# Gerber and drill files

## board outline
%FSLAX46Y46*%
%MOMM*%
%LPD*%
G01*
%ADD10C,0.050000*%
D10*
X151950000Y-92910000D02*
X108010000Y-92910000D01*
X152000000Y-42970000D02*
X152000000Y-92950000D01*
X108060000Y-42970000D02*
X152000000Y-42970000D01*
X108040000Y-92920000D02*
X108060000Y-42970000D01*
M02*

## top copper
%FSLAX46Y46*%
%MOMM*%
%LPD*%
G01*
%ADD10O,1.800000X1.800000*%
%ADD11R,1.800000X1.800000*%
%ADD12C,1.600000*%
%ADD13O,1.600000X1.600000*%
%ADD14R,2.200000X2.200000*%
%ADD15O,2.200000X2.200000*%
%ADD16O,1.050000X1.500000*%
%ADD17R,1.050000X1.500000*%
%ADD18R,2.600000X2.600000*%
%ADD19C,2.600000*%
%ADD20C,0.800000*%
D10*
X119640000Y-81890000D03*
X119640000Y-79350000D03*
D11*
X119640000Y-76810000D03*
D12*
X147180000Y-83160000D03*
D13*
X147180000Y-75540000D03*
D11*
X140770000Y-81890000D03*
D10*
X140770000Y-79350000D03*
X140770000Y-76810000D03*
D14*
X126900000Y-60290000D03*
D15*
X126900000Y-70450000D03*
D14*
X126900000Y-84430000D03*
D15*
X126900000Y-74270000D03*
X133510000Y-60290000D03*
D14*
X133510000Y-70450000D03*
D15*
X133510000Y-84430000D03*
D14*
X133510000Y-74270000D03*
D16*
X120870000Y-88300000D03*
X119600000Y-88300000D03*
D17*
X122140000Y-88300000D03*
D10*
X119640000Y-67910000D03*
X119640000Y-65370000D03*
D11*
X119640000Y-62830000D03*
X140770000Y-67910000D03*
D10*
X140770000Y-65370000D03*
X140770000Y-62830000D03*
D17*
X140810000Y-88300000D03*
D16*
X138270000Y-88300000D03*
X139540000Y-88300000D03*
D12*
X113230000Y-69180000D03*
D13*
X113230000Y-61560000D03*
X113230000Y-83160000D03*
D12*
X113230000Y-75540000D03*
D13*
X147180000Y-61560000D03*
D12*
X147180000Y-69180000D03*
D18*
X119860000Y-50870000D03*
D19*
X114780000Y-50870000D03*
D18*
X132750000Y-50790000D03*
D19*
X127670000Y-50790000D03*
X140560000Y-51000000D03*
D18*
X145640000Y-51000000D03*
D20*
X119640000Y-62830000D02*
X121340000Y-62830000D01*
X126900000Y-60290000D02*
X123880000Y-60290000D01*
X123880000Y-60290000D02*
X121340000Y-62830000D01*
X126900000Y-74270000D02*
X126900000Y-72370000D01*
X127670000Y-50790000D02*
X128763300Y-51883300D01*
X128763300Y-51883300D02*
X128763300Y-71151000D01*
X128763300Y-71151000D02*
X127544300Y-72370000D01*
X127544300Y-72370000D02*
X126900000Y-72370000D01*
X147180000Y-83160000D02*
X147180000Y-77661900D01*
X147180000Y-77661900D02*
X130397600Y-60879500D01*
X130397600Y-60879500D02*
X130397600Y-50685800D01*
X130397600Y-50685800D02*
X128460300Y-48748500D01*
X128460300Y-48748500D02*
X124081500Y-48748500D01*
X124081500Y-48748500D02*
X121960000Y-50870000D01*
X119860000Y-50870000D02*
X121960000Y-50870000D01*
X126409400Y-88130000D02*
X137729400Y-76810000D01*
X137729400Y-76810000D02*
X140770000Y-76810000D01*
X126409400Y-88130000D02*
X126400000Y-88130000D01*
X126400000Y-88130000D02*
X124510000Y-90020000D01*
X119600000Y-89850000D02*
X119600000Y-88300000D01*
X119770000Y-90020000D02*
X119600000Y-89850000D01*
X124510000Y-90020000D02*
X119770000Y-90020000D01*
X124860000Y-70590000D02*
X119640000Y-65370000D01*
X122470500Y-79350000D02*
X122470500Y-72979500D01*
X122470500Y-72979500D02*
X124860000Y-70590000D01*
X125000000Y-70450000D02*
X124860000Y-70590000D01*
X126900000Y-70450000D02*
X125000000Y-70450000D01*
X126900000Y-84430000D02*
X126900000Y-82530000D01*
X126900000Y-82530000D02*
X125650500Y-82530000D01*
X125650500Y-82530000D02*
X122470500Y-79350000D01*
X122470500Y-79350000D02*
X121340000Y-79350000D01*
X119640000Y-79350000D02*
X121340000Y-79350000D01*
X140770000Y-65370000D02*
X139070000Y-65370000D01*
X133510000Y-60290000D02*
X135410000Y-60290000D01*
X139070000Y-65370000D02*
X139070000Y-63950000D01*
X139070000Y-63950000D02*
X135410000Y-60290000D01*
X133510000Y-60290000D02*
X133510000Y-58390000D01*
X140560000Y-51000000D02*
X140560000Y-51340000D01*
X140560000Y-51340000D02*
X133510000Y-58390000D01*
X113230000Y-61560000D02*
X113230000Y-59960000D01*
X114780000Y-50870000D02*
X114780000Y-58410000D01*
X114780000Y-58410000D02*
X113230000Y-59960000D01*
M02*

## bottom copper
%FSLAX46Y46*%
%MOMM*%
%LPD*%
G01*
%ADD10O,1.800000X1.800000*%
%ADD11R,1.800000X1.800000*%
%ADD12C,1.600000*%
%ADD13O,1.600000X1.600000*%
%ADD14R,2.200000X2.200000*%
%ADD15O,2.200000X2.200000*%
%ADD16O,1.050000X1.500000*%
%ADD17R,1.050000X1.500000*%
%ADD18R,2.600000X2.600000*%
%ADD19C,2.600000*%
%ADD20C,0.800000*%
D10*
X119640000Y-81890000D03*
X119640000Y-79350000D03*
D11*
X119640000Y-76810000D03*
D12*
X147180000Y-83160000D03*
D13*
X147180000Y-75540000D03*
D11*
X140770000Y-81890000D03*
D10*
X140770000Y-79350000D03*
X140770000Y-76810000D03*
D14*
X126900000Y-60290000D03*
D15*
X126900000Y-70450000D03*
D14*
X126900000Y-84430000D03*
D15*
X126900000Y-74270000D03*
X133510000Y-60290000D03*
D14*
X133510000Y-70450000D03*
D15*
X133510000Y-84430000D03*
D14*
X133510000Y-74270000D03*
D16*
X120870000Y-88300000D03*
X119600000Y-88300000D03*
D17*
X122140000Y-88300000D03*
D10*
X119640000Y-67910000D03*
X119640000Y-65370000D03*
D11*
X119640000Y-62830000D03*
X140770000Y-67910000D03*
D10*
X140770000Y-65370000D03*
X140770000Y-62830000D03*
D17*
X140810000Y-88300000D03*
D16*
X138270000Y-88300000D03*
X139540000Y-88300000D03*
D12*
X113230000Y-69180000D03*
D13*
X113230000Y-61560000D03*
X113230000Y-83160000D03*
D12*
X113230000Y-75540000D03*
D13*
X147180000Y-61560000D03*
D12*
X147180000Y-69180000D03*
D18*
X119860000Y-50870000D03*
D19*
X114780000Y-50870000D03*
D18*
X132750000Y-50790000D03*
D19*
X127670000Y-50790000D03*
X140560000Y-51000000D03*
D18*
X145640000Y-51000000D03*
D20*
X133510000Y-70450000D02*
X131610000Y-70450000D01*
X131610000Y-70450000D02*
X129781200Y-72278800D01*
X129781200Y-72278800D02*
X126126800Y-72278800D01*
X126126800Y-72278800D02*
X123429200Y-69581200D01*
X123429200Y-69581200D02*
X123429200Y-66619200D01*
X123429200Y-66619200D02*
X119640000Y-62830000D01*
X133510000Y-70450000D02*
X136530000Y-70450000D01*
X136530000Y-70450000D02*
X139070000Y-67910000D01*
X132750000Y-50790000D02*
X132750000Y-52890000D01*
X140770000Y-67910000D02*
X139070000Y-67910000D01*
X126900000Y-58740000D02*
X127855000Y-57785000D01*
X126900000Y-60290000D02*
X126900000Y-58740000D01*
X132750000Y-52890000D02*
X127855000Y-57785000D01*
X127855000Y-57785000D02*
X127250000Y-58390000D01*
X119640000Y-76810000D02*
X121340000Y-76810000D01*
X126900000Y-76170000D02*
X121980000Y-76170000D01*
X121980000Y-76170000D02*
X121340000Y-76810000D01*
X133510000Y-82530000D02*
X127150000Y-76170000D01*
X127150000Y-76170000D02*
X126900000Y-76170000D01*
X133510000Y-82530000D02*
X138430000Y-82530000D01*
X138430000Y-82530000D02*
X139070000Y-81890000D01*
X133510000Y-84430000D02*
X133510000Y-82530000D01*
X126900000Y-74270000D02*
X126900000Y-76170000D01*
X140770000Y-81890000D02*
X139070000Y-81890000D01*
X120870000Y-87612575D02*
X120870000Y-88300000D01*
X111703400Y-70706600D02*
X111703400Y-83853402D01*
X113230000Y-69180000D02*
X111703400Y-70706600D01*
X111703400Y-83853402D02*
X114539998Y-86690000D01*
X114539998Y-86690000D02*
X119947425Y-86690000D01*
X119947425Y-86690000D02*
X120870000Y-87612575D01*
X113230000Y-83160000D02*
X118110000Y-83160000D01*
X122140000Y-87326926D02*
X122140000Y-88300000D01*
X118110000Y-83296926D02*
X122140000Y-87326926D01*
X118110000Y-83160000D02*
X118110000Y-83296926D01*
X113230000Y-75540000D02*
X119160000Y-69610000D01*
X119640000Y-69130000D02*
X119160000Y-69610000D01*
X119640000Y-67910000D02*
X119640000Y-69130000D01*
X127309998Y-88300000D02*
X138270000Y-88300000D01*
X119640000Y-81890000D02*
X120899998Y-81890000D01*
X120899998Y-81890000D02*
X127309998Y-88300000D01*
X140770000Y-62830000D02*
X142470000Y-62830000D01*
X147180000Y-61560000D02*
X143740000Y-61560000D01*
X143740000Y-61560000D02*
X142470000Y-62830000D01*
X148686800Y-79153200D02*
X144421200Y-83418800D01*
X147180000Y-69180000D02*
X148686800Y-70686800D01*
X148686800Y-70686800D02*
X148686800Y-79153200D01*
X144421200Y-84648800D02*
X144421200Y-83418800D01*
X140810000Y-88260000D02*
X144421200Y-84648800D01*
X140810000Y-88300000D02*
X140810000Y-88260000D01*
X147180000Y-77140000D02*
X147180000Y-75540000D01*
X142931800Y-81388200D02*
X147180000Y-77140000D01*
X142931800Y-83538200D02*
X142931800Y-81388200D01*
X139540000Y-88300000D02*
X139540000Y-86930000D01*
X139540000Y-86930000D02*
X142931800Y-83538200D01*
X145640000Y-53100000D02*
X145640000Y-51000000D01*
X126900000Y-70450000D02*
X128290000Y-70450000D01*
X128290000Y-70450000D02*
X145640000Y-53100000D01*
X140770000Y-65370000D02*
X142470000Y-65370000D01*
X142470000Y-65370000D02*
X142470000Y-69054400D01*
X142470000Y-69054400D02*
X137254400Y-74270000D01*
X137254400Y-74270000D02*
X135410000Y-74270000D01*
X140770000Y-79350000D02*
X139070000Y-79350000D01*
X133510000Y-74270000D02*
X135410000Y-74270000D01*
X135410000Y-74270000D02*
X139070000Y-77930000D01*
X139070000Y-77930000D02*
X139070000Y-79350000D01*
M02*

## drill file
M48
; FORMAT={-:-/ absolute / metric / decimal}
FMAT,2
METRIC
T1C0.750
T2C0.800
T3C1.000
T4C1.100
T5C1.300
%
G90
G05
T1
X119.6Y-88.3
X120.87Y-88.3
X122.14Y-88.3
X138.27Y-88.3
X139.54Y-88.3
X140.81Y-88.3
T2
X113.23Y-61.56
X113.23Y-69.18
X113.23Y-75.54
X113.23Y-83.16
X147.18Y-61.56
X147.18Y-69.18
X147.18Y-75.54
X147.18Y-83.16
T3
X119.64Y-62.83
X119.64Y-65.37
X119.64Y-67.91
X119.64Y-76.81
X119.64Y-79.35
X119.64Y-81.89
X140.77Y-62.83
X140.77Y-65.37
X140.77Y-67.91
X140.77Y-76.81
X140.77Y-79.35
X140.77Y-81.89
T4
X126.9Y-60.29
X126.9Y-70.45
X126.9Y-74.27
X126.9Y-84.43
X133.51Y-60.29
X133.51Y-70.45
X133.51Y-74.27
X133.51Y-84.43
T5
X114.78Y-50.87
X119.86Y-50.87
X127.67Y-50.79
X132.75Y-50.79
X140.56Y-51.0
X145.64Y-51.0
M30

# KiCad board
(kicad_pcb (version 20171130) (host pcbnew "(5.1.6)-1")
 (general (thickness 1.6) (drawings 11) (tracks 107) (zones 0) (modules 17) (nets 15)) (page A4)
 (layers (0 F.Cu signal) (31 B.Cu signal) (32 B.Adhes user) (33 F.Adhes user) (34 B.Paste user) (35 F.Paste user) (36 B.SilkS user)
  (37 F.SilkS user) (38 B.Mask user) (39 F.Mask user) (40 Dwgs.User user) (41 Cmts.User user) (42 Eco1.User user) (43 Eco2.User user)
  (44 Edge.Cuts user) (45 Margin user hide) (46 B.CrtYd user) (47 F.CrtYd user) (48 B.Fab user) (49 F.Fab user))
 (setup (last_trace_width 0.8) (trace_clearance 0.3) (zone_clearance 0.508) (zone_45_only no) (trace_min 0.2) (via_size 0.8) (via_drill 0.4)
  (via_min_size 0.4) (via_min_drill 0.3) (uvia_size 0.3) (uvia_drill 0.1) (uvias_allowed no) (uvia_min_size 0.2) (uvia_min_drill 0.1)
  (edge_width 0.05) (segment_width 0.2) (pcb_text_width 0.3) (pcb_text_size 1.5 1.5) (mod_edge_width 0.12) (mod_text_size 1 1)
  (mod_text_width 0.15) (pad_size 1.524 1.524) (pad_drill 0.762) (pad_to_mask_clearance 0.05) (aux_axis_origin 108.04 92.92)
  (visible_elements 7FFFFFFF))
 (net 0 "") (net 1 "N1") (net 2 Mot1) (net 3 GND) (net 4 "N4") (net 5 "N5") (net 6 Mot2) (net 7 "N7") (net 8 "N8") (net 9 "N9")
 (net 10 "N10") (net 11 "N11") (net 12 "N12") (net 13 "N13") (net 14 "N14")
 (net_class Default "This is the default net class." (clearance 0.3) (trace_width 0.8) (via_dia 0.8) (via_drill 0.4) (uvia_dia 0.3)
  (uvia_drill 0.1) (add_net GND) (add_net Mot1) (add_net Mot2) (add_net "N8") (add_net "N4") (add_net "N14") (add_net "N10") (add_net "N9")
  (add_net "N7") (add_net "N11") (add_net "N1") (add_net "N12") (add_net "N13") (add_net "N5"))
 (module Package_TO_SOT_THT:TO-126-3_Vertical (layer F.Cu) (at 119.64 76.81 270)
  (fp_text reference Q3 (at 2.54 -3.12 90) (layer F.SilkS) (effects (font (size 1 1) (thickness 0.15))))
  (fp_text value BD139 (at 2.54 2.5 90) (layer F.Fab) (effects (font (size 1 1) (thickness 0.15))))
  (pad 3 thru_hole oval (at 5.08 0 270) (size 1.8 1.8) (drill 1) (layers *.Cu *.Mask) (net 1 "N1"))
  (pad 2 thru_hole oval (at 2.54 0 270) (size 1.8 1.8) (drill 1) (layers *.Cu *.Mask) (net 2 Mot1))
  (pad 1 thru_hole rect (at 0 0 270) (size 1.8 1.8) (drill 1) (layers *.Cu *.Mask) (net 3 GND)))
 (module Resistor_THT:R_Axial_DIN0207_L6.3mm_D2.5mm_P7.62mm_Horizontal (layer F.Cu) (at 147.18 83.16 90)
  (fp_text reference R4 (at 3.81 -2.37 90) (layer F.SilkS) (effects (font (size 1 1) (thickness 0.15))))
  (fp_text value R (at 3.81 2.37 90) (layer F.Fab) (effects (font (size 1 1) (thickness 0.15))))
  (pad 1 thru_hole circle (at 0 0 90) (size 1.6 1.6) (drill 0.8) (layers *.Cu *.Mask) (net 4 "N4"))
  (pad 2 thru_hole oval (at 7.62 0 90) (size 1.6 1.6) (drill 0.8) (layers *.Cu *.Mask) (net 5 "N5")))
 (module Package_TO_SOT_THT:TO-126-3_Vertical (layer F.Cu) (at 140.77 81.89 90)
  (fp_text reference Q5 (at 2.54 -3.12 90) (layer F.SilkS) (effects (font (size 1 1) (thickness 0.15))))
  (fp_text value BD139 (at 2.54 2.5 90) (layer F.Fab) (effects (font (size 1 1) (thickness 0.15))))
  (pad 1 thru_hole rect (at 0 0 90) (size 1.8 1.8) (drill 1) (layers *.Cu *.Mask) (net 3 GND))
  (pad 2 thru_hole oval (at 2.54 0 90) (size 1.8 1.8) (drill 1) (layers *.Cu *.Mask) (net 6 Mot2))
  (pad 3 thru_hole oval (at 5.08 0 90) (size 1.8 1.8) (drill 1) (layers *.Cu *.Mask) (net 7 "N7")))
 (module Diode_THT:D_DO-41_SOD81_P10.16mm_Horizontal (layer F.Cu) (at 126.9 60.29 270)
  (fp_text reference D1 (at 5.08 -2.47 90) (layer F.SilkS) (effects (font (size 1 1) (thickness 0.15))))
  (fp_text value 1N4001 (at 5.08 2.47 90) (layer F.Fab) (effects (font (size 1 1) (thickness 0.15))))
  (pad 1 thru_hole rect (at 0 0 270) (size 2.2 2.2) (drill 1.1) (layers *.Cu *.Mask) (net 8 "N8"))
  (pad 2 thru_hole oval (at 10.16 0 270) (size 2.2 2.2) (drill 1.1) (layers *.Cu *.Mask) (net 2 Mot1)))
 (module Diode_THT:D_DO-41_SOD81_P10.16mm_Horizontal (layer F.Cu) (at 126.9 84.43 90)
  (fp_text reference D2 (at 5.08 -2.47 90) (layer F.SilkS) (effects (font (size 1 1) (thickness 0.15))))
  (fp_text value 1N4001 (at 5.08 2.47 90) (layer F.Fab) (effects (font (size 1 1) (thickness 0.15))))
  (pad 1 thru_hole rect (at 0 0 90) (size 2.2 2.2) (drill 1.1) (layers *.Cu *.Mask) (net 2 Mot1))
  (pad 2 thru_hole oval (at 10.16 0 90) (size 2.2 2.2) (drill 1.1) (layers *.Cu *.Mask) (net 3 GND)))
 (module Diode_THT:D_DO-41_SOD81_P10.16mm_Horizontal (layer F.Cu) (at 133.51 70.45 90)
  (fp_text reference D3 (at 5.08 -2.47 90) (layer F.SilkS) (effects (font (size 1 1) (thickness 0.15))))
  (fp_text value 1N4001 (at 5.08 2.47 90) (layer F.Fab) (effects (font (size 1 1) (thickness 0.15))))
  (pad 2 thru_hole oval (at 10.16 0 90) (size 2.2 2.2) (drill 1.1) (layers *.Cu *.Mask) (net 6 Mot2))
  (pad 1 thru_hole rect (at 0 0 90) (size 2.2 2.2) (drill 1.1) (layers *.Cu *.Mask) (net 8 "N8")))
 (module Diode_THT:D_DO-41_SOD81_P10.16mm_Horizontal (layer F.Cu) (at 133.51 74.27 270)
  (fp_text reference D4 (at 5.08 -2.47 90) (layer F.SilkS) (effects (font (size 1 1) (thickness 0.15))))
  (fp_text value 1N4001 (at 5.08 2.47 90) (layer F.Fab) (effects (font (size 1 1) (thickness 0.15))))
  (pad 2 thru_hole oval (at 10.16 0 270) (size 2.2 2.2) (drill 1.1) (layers *.Cu *.Mask) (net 3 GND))
  (pad 1 thru_hole rect (at 0 0 270) (size 2.2 2.2) (drill 1.1) (layers *.Cu *.Mask) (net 6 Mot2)))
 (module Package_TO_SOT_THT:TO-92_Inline (layer F.Cu) (at 122.14 88.3 180)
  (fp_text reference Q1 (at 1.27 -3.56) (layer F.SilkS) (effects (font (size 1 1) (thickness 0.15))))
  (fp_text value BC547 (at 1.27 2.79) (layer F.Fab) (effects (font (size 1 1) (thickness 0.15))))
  (pad 2 thru_hole oval (at 1.27 0 180) (size 1.05 1.5) (drill 0.75) (layers *.Cu *.Mask) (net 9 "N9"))
  (pad 3 thru_hole oval (at 2.54 0 180) (size 1.05 1.5) (drill 0.75) (layers *.Cu *.Mask) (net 7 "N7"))
  (pad 1 thru_hole rect (at 0 0 180) (size 1.05 1.5) (drill 0.75) (layers *.Cu *.Mask) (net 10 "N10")))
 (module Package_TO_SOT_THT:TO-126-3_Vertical (layer F.Cu) (at 119.64 62.83 270)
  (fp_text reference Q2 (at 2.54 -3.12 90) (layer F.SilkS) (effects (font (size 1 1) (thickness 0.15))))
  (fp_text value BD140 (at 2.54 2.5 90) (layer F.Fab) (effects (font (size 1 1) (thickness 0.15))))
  (pad 3 thru_hole oval (at 5.08 0 270) (size 1.8 1.8) (drill 1) (layers *.Cu *.Mask) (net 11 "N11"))
  (pad 2 thru_hole oval (at 2.54 0 270) (size 1.8 1.8) (drill 1) (layers *.Cu *.Mask) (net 2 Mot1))
  (pad 1 thru_hole rect (at 0 0 270) (size 1.8 1.8) (drill 1) (layers *.Cu *.Mask) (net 8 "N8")))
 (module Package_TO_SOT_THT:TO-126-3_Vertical (layer F.Cu) (at 140.77 67.91 90)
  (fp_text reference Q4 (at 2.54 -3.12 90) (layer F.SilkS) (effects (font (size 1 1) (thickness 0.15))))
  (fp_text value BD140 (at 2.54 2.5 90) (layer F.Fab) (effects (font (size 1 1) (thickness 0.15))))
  (pad 1 thru_hole rect (at 0 0 90) (size 1.8 1.8) (drill 1) (layers *.Cu *.Mask) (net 8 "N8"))
  (pad 2 thru_hole oval (at 2.54 0 90) (size 1.8 1.8) (drill 1) (layers *.Cu *.Mask) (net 6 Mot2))
  (pad 3 thru_hole oval (at 5.08 0 90) (size 1.8 1.8) (drill 1) (layers *.Cu *.Mask) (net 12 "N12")))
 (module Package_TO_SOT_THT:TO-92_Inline (layer F.Cu) (at 140.81 88.3 180)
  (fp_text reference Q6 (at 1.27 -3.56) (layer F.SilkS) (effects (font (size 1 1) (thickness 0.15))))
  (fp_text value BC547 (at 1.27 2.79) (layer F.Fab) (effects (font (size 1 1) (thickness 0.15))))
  (pad 1 thru_hole rect (at 0 0 180) (size 1.05 1.5) (drill 0.75) (layers *.Cu *.Mask) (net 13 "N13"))
  (pad 3 thru_hole oval (at 2.54 0 180) (size 1.05 1.5) (drill 0.75) (layers *.Cu *.Mask) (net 1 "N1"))
  (pad 2 thru_hole oval (at 1.27 0 180) (size 1.05 1.5) (drill 0.75) (layers *.Cu *.Mask) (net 5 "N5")))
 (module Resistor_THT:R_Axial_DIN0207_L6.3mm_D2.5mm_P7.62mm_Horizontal (layer F.Cu) (at 113.23 69.18 90)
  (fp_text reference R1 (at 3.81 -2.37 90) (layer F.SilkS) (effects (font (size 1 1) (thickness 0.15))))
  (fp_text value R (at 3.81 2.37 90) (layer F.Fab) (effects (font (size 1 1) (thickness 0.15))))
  (pad 1 thru_hole circle (at 0 0 90) (size 1.6 1.6) (drill 0.8) (layers *.Cu *.Mask) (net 9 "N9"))
  (pad 2 thru_hole oval (at 7.62 0 90) (size 1.6 1.6) (drill 0.8) (layers *.Cu *.Mask) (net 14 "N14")))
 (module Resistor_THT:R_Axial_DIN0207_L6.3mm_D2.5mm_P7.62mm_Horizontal (layer F.Cu) (at 113.23 75.54 270)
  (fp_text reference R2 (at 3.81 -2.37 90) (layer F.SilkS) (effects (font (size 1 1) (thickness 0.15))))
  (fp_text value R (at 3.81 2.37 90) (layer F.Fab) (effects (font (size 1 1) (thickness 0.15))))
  (pad 2 thru_hole oval (at 7.62 0 270) (size 1.6 1.6) (drill 0.8) (layers *.Cu *.Mask) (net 10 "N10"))
  (pad 1 thru_hole circle (at 0 0 270) (size 1.6 1.6) (drill 0.8) (layers *.Cu *.Mask) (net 11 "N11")))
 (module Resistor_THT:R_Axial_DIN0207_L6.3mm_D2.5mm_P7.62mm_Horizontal (layer F.Cu) (at 147.18 69.18 90)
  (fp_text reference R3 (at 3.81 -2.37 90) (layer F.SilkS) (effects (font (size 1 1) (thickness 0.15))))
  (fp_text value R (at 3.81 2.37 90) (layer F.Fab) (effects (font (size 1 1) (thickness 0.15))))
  (pad 2 thru_hole oval (at 7.62 0 90) (size 1.6 1.6) (drill 0.8) (layers *.Cu *.Mask) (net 12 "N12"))
  (pad 1 thru_hole circle (at 0 0 90) (size 1.6 1.6) (drill 0.8) (layers *.Cu *.Mask) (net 13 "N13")))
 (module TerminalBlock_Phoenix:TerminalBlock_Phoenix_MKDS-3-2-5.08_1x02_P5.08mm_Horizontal (layer F.Cu) (at 119.86 50.87 180)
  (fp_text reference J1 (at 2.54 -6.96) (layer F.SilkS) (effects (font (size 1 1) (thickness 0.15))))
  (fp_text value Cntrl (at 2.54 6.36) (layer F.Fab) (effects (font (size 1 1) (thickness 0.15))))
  (pad 1 thru_hole rect (at 0 0 180) (size 2.6 2.6) (drill 1.3) (layers *.Cu *.Mask) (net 4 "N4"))
  (pad 2 thru_hole circle (at 5.08 0 180) (size 2.6 2.6) (drill 1.3) (layers *.Cu *.Mask) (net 14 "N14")))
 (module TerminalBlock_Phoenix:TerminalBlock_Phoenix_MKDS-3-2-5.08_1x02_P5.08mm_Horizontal (layer F.Cu) (at 132.75 50.79 180)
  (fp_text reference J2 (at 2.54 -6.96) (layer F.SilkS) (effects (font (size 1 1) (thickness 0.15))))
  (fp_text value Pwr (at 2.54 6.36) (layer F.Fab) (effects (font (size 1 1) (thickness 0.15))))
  (pad 1 thru_hole rect (at 0 0 180) (size 2.6 2.6) (drill 1.3) (layers *.Cu *.Mask) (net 8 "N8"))
  (pad 2 thru_hole circle (at 5.08 0 180) (size 2.6 2.6) (drill 1.3) (layers *.Cu *.Mask) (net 3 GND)))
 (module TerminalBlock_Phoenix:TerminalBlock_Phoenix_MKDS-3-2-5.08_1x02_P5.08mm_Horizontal (layer F.Cu) (at 145.64 51 180)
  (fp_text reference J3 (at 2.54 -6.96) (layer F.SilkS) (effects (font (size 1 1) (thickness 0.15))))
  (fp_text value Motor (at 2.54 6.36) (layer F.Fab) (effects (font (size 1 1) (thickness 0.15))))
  (pad 2 thru_hole circle (at 5.08 0 180) (size 2.6 2.6) (drill 1.3) (layers *.Cu *.Mask) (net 6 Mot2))
  (pad 1 thru_hole rect (at 0 0 180) (size 2.6 2.6) (drill 1.3) (layers *.Cu *.Mask) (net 2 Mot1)))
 (gr_line (start 151.95 92.91) (end 108.01 92.91) (layer Edge.Cuts) (width 0.05))
 (gr_line (start 152 42.97) (end 152 92.95) (layer Edge.Cuts) (width 0.05))
 (gr_line (start 108.06 42.97) (end 152 42.97) (layer Edge.Cuts) (width 0.05))
 (gr_line (start 108.04 92.92) (end 108.06 42.97) (layer Edge.Cuts) (width 0.05))
 (segment (start 133.51 70.45) (end 131.61 70.45) (width 0.8) (layer B.Cu) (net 8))
 (segment (start 131.61 70.45) (end 129.7812 72.2788) (width 0.8) (layer B.Cu) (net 8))
 (segment (start 129.7812 72.2788) (end 126.1268 72.2788) (width 0.8) (layer B.Cu) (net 8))
 (segment (start 126.1268 72.2788) (end 123.4292 69.5812) (width 0.8) (layer B.Cu) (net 8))
 (segment (start 123.4292 69.5812) (end 123.4292 66.6192) (width 0.8) (layer B.Cu) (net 8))
 (segment (start 123.4292 66.6192) (end 119.64 62.83) (width 0.8) (layer B.Cu) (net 8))
 (segment (start 133.51 70.45) (end 136.53 70.45) (width 0.8) (layer B.Cu) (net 8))
 (segment (start 136.53 70.45) (end 139.07 67.91) (width 0.8) (layer B.Cu) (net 8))
 (segment (start 132.75 50.79) (end 132.75 52.89) (width 0.8) (layer B.Cu) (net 8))
 (segment (start 119.64 62.83) (end 121.34 62.83) (width 0.8) (layer F.Cu) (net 8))
 (segment (start 126.9 60.29) (end 123.88 60.29) (width 0.8) (layer F.Cu) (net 8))
 (segment (start 123.88 60.29) (end 121.34 62.83) (width 0.8) (layer F.Cu) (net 8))
 (segment (start 140.77 67.91) (end 139.07 67.91) (width 0.8) (layer B.Cu) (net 8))
 (segment (start 126.9 58.74) (end 127.855 57.785) (width 0.8) (layer B.Cu) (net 8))
 (segment (start 126.9 60.29) (end 126.9 58.74) (width 0.8) (layer B.Cu) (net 8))
 (segment (start 132.75 52.89) (end 127.855 57.785) (width 0.8) (layer B.Cu) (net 8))
 (segment (start 127.855 57.785) (end 127.25 58.39) (width 0.8) (layer B.Cu) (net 8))
 (segment (start 126.9 74.27) (end 126.9 72.37) (width 0.8) (layer F.Cu) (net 3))
 (segment (start 127.67 50.79) (end 128.7633 51.8833) (width 0.8) (layer F.Cu) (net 3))
 (segment (start 128.7633 51.8833) (end 128.7633 71.151) (width 0.8) (layer F.Cu) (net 3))
 (segment (start 128.7633 71.151) (end 127.5443 72.37) (width 0.8) (layer F.Cu) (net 3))
 (segment (start 127.5443 72.37) (end 126.9 72.37) (width 0.8) (layer F.Cu) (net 3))
 (segment (start 119.64 76.81) (end 121.34 76.81) (width 0.8) (layer B.Cu) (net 3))
 (segment (start 126.9 76.17) (end 121.98 76.17) (width 0.8) (layer B.Cu) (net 3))
 (segment (start 121.98 76.17) (end 121.34 76.81) (width 0.8) (layer B.Cu) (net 3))
 (segment (start 133.51 82.53) (end 127.15 76.17) (width 0.8) (layer B.Cu) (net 3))
 (segment (start 127.15 76.17) (end 126.9 76.17) (width 0.8) (layer B.Cu) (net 3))
 (segment (start 133.51 82.53) (end 138.43 82.53) (width 0.8) (layer B.Cu) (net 3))
 (segment (start 138.43 82.53) (end 139.07 81.89) (width 0.8) (layer B.Cu) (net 3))
 (segment (start 133.51 84.43) (end 133.51 82.53) (width 0.8) (layer B.Cu) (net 3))
 (segment (start 126.9 74.27) (end 126.9 76.17) (width 0.8) (layer B.Cu) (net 3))
 (segment (start 140.77 81.89) (end 139.07 81.89) (width 0.8) (layer B.Cu) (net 3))
 (segment (start 147.18 83.16) (end 147.18 77.6619) (width 0.8) (layer F.Cu) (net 4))
 (segment (start 147.18 77.6619) (end 130.3976 60.8795) (width 0.8) (layer F.Cu) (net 4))
 (segment (start 130.3976 60.8795) (end 130.3976 50.6858) (width 0.8) (layer F.Cu) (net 4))
 (segment (start 130.3976 50.6858) (end 128.4603 48.7485) (width 0.8) (layer F.Cu) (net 4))
 (segment (start 128.4603 48.7485) (end 124.0815 48.7485) (width 0.8) (layer F.Cu) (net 4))
 (segment (start 124.0815 48.7485) (end 121.96 50.87) (width 0.8) (layer F.Cu) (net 4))
 (segment (start 119.86 50.87) (end 121.96 50.87) (width 0.8) (layer F.Cu) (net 4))
 (segment (start 120.87 87.612575) (end 120.87 88.3) (width 0.8) (layer B.Cu) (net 9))
 (segment (start 111.7034 70.7066) (end 111.7034 83.853402) (width 0.8) (layer B.Cu) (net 9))
 (segment (start 113.23 69.18) (end 111.7034 70.7066) (width 0.8) (layer B.Cu) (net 9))
 (segment (start 111.7034 83.853402) (end 114.539998 86.69) (width 0.8) (layer B.Cu) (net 9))
 (segment (start 114.539998 86.69) (end 119.947425 86.69) (width 0.8) (layer B.Cu) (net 9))
 (segment (start 119.947425 86.69) (end 120.87 87.612575) (width 0.8) (layer B.Cu) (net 9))
 (segment (start 126.4094 88.13) (end 137.7294 76.81) (width 0.8) (layer F.Cu) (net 7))
 (segment (start 137.7294 76.81) (end 140.77 76.81) (width 0.8) (layer F.Cu) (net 7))
 (segment (start 126.4094 88.13) (end 126.4 88.13) (width 0.8) (layer F.Cu) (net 7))
 (segment (start 126.4 88.13) (end 124.51 90.02) (width 0.8) (layer F.Cu) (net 7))
 (segment (start 119.6 89.85) (end 119.6 88.3) (width 0.8) (layer F.Cu) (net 7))
 (segment (start 119.77 90.02) (end 119.6 89.85) (width 0.8) (layer F.Cu) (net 7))
 (segment (start 124.51 90.02) (end 119.77 90.02) (width 0.8) (layer F.Cu) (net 7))
 (segment (start 113.23 83.16) (end 118.11 83.16) (width 0.8) (layer B.Cu) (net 10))
 (segment (start 122.14 87.326926) (end 122.14 88.3) (width 0.8) (layer B.Cu) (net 10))
 (segment (start 118.11 83.296926) (end 122.14 87.326926) (width 0.8) (layer B.Cu) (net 10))
 (segment (start 118.11 83.16) (end 118.11 83.296926) (width 0.8) (layer B.Cu) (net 10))
 (segment (start 113.23 75.54) (end 119.16 69.61) (width 0.8) (layer B.Cu) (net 11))
 (segment (start 119.64 69.13) (end 119.16 69.61) (width 0.8) (layer B.Cu) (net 11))
 (segment (start 119.64 67.91) (end 119.64 69.13) (width 0.8) (layer B.Cu) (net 11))
 (segment (start 127.309998 88.3) (end 138.27 88.3) (width 0.8) (layer B.Cu) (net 1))
 (segment (start 119.64 81.89) (end 120.899998 81.89) (width 0.8) (layer B.Cu) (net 1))
 (segment (start 120.899998 81.89) (end 127.309998 88.3) (width 0.8) (layer B.Cu) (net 1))
 (segment (start 140.77 62.83) (end 142.47 62.83) (width 0.8) (layer B.Cu) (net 12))
 (segment (start 147.18 61.56) (end 143.74 61.56) (width 0.8) (layer B.Cu) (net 12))
 (segment (start 143.74 61.56) (end 142.47 62.83) (width 0.8) (layer B.Cu) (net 12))
 (segment (start 148.6868 79.1532) (end 144.4212 83.4188) (width 0.8) (layer B.Cu) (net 13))
 (segment (start 147.18 69.18) (end 148.6868 70.6868) (width 0.8) (layer B.Cu) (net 13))
 (segment (start 148.6868 70.6868) (end 148.6868 79.1532) (width 0.8) (layer B.Cu) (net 13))
 (segment (start 144.4212 84.6488) (end 144.4212 83.4188) (width 0.8) (layer B.Cu) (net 13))
 (segment (start 140.81 88.26) (end 144.4212 84.6488) (width 0.8) (layer B.Cu) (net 13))
 (segment (start 140.81 88.3) (end 140.81 88.26) (width 0.8) (layer B.Cu) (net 13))
 (segment (start 147.18 77.14) (end 147.18 75.54) (width 0.8) (layer B.Cu) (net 5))
 (segment (start 142.9318 81.3882) (end 147.18 77.14) (width 0.8) (layer B.Cu) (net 5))
 (segment (start 142.9318 83.5382) (end 142.9318 81.3882) (width 0.8) (layer B.Cu) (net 5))
 (segment (start 139.54 88.3) (end 139.54 86.93) (width 0.8) (layer B.Cu) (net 5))
 (segment (start 139.54 86.93) (end 142.9318 83.5382) (width 0.8) (layer B.Cu) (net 5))
 (segment (start 124.86 70.59) (end 119.64 65.37) (width 0.8) (layer F.Cu) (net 2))
 (segment (start 122.4705 79.35) (end 122.4705 72.9795) (width 0.8) (layer F.Cu) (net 2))
 (segment (start 122.4705 72.9795) (end 124.86 70.59) (width 0.8) (layer F.Cu) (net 2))
 (segment (start 125 70.45) (end 124.86 70.59) (width 0.8) (layer F.Cu) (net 2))
 (segment (start 126.9 70.45) (end 125 70.45) (width 0.8) (layer F.Cu) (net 2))
 (segment (start 126.9 84.43) (end 126.9 82.53) (width 0.8) (layer F.Cu) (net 2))
 (segment (start 126.9 82.53) (end 125.6505 82.53) (width 0.8) (layer F.Cu) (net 2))
 (segment (start 125.6505 82.53) (end 122.4705 79.35) (width 0.8) (layer F.Cu) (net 2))
 (segment (start 122.4705 79.35) (end 121.34 79.35) (width 0.8) (layer F.Cu) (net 2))
 (segment (start 119.64 79.35) (end 121.34 79.35) (width 0.8) (layer F.Cu) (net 2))
 (segment (start 145.64 53.1) (end 145.64 51) (width 0.8) (layer B.Cu) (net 2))
 (segment (start 126.9 70.45) (end 128.29 70.45) (width 0.8) (layer B.Cu) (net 2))
 (segment (start 128.29 70.45) (end 145.64 53.1) (width 0.8) (layer B.Cu) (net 2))
 (segment (start 140.77 65.37) (end 139.07 65.37) (width 0.8) (layer F.Cu) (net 6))
 (segment (start 133.51 60.29) (end 135.41 60.29) (width 0.8) (layer F.Cu) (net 6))
 (segment (start 139.07 65.37) (end 139.07 63.95) (width 0.8) (layer F.Cu) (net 6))
 (segment (start 139.07 63.95) (end 135.41 60.29) (width 0.8) (layer F.Cu) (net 6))
 (segment (start 133.51 60.29) (end 133.51 58.39) (width 0.8) (layer F.Cu) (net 6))
 (segment (start 140.56 51) (end 140.56 51.34) (width 0.8) (layer F.Cu) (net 6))
 (segment (start 140.56 51.34) (end 133.51 58.39) (width 0.8) (layer F.Cu) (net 6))
 (segment (start 140.77 65.37) (end 142.47 65.37) (width 0.8) (layer B.Cu) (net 6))
 (segment (start 142.47 65.37) (end 142.47 69.0544) (width 0.8) (layer B.Cu) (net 6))
 (segment (start 142.47 69.0544) (end 137.2544 74.27) (width 0.8) (layer B.Cu) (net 6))
 (segment (start 137.2544 74.27) (end 135.41 74.27) (width 0.8) (layer B.Cu) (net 6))
 (segment (start 140.77 79.35) (end 139.07 79.35) (width 0.8) (layer B.Cu) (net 6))
 (segment (start 133.51 74.27) (end 135.41 74.27) (width 0.8) (layer B.Cu) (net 6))
 (segment (start 135.41 74.27) (end 139.07 77.93) (width 0.8) (layer B.Cu) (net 6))
 (segment (start 139.07 77.93) (end 139.07 79.35) (width 0.8) (layer B.Cu) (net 6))
 (segment (start 113.23 61.56) (end 113.23 59.96) (width 0.8) (layer F.Cu) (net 14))
 (segment (start 114.78 50.87) (end 114.78 58.41) (width 0.8) (layer F.Cu) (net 14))
 (segment (start 114.78 58.41) (end 113.23 59.96) (width 0.8) (layer F.Cu) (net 14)))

